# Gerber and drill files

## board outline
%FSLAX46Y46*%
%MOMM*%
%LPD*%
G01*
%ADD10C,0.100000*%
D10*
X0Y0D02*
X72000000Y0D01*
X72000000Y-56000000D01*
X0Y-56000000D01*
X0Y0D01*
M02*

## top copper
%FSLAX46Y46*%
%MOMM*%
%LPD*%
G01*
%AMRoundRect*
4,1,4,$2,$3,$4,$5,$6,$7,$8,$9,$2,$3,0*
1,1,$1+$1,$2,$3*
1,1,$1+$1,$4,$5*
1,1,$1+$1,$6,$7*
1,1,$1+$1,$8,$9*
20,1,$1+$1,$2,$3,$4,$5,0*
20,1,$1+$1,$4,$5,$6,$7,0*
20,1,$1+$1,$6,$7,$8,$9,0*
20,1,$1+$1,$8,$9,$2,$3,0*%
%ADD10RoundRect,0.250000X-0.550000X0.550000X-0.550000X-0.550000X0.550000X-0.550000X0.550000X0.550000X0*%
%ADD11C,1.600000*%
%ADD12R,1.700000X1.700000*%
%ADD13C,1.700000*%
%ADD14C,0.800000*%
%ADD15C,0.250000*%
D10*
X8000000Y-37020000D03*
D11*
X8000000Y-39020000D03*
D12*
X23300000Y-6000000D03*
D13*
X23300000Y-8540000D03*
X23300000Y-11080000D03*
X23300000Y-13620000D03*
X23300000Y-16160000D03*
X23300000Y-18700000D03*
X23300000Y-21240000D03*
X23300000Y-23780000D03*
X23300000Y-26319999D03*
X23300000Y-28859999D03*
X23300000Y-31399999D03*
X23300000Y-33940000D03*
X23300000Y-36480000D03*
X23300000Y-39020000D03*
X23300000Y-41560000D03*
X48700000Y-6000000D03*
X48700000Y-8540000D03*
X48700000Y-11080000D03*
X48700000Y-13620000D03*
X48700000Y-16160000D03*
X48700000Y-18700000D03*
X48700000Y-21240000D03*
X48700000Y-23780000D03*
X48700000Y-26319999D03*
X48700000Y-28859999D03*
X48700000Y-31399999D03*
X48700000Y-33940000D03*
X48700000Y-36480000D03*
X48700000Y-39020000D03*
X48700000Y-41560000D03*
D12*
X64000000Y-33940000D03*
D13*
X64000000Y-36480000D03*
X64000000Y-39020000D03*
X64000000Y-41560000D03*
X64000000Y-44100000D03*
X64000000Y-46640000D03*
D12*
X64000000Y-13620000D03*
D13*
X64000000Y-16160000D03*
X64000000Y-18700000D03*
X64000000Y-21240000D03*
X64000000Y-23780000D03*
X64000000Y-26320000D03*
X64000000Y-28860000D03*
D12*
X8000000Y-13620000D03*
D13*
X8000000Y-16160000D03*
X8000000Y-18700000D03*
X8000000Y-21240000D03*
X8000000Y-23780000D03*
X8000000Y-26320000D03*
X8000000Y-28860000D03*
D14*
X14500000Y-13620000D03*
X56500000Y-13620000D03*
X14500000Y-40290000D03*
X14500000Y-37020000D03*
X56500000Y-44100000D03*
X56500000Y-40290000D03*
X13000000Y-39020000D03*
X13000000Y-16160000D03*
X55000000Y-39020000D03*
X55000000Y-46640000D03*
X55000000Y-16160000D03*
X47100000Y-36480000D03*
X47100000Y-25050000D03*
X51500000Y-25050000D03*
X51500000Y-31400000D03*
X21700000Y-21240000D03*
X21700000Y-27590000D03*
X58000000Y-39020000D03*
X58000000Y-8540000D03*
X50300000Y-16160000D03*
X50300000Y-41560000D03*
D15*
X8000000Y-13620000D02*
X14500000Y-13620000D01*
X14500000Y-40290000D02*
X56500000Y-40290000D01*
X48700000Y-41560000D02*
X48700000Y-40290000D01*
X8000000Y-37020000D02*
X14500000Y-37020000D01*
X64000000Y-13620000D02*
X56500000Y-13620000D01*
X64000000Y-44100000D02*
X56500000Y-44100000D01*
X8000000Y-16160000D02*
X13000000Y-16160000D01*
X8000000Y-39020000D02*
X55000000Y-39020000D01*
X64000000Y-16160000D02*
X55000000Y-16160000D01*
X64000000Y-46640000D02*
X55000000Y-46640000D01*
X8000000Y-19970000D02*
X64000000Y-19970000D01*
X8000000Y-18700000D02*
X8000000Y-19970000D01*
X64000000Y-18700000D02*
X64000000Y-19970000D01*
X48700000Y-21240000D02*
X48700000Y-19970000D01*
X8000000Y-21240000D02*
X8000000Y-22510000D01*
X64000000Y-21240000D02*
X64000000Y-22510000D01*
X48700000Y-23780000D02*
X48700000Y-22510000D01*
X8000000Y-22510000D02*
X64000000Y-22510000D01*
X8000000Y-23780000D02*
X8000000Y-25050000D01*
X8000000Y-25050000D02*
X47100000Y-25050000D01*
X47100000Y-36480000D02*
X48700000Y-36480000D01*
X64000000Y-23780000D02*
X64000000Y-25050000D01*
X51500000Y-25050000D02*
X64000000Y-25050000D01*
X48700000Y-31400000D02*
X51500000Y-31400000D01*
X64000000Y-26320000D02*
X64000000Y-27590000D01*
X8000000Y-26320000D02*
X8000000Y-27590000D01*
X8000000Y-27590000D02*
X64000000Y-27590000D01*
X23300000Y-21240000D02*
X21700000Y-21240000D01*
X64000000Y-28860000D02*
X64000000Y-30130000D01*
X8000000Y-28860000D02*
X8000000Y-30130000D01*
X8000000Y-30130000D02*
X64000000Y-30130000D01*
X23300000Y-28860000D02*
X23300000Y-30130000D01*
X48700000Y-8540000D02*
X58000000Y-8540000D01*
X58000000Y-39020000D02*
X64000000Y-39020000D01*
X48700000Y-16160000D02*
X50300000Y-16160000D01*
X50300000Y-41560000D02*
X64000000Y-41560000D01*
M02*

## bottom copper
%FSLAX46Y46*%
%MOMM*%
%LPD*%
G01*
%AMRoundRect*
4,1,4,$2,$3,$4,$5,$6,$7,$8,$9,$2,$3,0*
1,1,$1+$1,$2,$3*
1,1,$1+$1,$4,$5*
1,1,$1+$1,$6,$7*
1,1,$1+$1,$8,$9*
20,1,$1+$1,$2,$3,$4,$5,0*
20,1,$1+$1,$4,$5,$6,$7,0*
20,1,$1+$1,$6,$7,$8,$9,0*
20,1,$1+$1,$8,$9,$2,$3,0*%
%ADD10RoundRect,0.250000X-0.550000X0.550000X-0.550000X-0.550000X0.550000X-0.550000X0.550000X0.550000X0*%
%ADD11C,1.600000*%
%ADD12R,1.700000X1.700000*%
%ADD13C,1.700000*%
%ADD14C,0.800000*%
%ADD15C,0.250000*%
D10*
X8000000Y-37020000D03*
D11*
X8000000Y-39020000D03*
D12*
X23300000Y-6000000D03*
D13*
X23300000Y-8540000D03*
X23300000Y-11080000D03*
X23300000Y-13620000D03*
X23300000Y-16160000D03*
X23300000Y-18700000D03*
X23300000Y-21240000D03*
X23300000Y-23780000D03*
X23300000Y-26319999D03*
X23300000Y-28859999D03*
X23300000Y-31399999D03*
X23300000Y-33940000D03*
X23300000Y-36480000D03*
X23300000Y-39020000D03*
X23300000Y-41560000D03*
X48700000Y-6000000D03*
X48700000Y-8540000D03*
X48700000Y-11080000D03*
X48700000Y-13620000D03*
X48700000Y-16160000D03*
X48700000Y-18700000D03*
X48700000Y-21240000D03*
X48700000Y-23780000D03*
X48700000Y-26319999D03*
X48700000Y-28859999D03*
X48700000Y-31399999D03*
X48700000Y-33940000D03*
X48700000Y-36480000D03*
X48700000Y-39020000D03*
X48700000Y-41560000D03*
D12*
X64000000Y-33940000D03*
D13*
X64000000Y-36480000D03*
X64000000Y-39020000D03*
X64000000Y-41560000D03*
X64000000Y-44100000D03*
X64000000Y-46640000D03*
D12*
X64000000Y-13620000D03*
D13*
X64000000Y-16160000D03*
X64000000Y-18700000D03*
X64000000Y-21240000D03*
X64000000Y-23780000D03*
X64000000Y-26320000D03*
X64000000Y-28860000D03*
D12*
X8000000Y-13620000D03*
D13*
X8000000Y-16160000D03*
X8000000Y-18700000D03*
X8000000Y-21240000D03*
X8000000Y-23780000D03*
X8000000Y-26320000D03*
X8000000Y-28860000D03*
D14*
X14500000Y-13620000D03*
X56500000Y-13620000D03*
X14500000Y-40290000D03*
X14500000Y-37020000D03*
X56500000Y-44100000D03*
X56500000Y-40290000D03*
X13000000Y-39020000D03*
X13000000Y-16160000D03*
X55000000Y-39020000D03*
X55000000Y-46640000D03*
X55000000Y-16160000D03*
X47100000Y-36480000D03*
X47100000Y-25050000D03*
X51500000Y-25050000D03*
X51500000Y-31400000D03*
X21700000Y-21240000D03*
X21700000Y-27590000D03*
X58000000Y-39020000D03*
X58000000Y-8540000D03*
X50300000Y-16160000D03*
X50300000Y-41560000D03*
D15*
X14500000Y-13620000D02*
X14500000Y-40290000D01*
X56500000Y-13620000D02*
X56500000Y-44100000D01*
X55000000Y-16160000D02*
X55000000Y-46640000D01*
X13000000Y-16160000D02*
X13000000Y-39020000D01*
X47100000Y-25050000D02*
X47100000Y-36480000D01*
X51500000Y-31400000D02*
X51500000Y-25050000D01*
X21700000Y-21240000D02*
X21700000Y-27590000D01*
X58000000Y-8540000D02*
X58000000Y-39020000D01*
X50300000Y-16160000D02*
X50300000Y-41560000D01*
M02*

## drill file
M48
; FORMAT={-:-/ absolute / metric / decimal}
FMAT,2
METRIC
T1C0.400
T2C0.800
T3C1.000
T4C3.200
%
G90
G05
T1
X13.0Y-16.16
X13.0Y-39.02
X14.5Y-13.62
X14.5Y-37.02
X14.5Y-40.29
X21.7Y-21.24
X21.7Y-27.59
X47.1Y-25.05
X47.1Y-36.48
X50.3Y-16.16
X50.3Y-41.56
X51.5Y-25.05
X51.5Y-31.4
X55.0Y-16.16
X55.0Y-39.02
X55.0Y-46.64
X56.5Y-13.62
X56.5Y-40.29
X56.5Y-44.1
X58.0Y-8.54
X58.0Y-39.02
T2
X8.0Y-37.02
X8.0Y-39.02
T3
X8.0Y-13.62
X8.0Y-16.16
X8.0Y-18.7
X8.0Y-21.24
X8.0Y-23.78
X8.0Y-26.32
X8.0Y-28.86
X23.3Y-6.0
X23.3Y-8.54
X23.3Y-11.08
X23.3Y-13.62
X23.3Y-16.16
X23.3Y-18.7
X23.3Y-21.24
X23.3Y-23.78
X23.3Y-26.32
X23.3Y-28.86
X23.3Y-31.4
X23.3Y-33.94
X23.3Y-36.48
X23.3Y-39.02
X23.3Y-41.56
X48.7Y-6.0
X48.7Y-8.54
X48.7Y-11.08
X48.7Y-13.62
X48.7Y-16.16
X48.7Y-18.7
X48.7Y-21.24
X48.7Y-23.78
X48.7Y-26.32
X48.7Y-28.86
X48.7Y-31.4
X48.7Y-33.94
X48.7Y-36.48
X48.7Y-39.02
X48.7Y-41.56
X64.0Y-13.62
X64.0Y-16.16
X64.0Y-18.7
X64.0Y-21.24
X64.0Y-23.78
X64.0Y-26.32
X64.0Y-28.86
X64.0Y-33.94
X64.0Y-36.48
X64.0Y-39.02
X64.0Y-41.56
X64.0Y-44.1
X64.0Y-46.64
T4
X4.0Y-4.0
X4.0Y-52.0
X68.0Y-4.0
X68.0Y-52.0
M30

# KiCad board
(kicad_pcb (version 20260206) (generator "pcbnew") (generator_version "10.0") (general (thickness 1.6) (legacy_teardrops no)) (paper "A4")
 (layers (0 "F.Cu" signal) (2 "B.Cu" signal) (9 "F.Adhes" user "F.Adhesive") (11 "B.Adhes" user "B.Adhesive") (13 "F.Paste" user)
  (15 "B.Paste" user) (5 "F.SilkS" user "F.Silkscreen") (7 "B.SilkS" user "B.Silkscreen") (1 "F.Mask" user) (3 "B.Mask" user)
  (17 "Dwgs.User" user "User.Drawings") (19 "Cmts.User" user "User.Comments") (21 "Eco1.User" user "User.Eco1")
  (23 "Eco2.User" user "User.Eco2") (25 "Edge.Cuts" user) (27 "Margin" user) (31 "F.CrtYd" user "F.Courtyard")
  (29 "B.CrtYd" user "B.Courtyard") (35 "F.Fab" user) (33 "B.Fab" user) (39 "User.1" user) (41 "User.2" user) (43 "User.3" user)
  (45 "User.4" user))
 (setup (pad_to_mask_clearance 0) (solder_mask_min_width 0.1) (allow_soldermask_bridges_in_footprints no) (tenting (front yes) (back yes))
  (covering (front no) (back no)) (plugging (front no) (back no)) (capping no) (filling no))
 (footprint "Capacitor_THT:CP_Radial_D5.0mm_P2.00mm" (layer "F.Cu") (at 8 37.02 -90)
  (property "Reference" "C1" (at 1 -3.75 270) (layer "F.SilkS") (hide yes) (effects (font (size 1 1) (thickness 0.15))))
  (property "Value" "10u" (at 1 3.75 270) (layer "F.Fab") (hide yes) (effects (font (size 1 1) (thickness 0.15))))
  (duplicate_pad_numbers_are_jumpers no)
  (pad "1" thru_hole roundrect (at 0 0 270) (size 1.6 1.6) (drill 0.8) (layers "*.Cu" "*.Mask") (remove_unused_layers no)
   (roundrect_rratio 0.15625) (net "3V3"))
  (pad "2" thru_hole circle (at 2 0 270) (size 1.6 1.6) (drill 0.8) (layers "*.Cu" "*.Mask") (remove_unused_layers no) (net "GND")))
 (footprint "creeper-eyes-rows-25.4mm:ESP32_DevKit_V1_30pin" (layer "F.Cu") (at 36 23.78)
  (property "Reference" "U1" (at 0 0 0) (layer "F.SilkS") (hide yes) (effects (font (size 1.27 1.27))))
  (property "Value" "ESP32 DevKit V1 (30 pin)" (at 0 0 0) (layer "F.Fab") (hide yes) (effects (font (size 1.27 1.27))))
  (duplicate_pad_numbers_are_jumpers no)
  (pad "1" thru_hole rect (at -12.7 -17.78) (size 1.7 1.7) (drill 1) (layers "*.Cu" "*.Mask") (remove_unused_layers no)
   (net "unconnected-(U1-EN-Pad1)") (thermal_bridge_angle 45))
  (pad "2" thru_hole circle (at -12.7 -15.24) (size 1.7 1.7) (drill 1) (layers "*.Cu" "*.Mask") (remove_unused_layers no)
   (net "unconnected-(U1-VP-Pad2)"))
  (pad "3" thru_hole circle (at -12.7 -12.7) (size 1.7 1.7) (drill 1) (layers "*.Cu" "*.Mask") (remove_unused_layers no)
   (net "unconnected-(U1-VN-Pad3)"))
  (pad "4" thru_hole circle (at -12.7 -10.16) (size 1.7 1.7) (drill 1) (layers "*.Cu" "*.Mask") (remove_unused_layers no)
   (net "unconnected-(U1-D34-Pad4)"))
  (pad "5" thru_hole circle (at -12.7 -7.62) (size 1.7 1.7) (drill 1) (layers "*.Cu" "*.Mask") (remove_unused_layers no)
   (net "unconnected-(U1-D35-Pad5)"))
  (pad "6" thru_hole circle (at -12.7 -5.08) (size 1.7 1.7) (drill 1) (layers "*.Cu" "*.Mask") (remove_unused_layers no)
   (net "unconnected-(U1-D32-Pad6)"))
  (pad "7" thru_hole circle (at -12.7 -2.54) (size 1.7 1.7) (drill 1) (layers "*.Cu" "*.Mask") (remove_unused_layers no) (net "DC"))
  (pad "8" thru_hole circle (at -12.7 0) (size 1.7 1.7) (drill 1) (layers "*.Cu" "*.Mask") (remove_unused_layers no)
   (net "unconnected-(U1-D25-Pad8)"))
  (pad "9" thru_hole circle (at -12.7 2.539999) (size 1.7 1.7) (drill 1) (layers "*.Cu" "*.Mask") (remove_unused_layers no)
   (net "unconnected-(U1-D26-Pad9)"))
  (pad "10" thru_hole circle (at -12.7 5.079999) (size 1.7 1.7) (drill 1) (layers "*.Cu" "*.Mask") (remove_unused_layers no) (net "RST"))
  (pad "11" thru_hole circle (at -12.7 7.619999) (size 1.7 1.7) (drill 1) (layers "*.Cu" "*.Mask") (remove_unused_layers no)
   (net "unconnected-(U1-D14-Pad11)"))
  (pad "12" thru_hole circle (at -12.7 10.16) (size 1.7 1.7) (drill 1) (layers "*.Cu" "*.Mask") (remove_unused_layers no)
   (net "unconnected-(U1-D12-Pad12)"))
  (pad "13" thru_hole circle (at -12.7 12.7) (size 1.7 1.7) (drill 1) (layers "*.Cu" "*.Mask") (remove_unused_layers no)
   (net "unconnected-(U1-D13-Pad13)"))
  (pad "14" thru_hole circle (at -12.7 15.24) (size 1.7 1.7) (drill 1) (layers "*.Cu" "*.Mask") (remove_unused_layers no) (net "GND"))
  (pad "15" thru_hole circle (at -12.7 17.78) (size 1.7 1.7) (drill 1) (layers "*.Cu" "*.Mask") (remove_unused_layers no)
   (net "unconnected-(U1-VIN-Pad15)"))
  (pad "16" thru_hole circle (at 12.7 -17.78) (size 1.7 1.7) (drill 1) (layers "*.Cu" "*.Mask") (remove_unused_layers no)
   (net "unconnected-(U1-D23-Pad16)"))
  (pad "17" thru_hole circle (at 12.7 -15.24) (size 1.7 1.7) (drill 1) (layers "*.Cu" "*.Mask") (remove_unused_layers no) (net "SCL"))
  (pad "18" thru_hole circle (at 12.7 -12.7) (size 1.7 1.7) (drill 1) (layers "*.Cu" "*.Mask") (remove_unused_layers no)
   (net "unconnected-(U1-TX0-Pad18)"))
  (pad "19" thru_hole circle (at 12.7 -10.16) (size 1.7 1.7) (drill 1) (layers "*.Cu" "*.Mask") (remove_unused_layers no)
   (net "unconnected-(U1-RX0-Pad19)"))
  (pad "20" thru_hole circle (at 12.7 -7.62) (size 1.7 1.7) (drill 1) (layers "*.Cu" "*.Mask") (remove_unused_layers no) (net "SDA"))
  (pad "21" thru_hole circle (at 12.7 -5.08) (size 1.7 1.7) (drill 1) (layers "*.Cu" "*.Mask") (remove_unused_layers no)
   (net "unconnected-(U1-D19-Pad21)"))
  (pad "22" thru_hole circle (at 12.7 -2.54) (size 1.7 1.7) (drill 1) (layers "*.Cu" "*.Mask") (remove_unused_layers no) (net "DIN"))
  (pad "23" thru_hole circle (at 12.7 0) (size 1.7 1.7) (drill 1) (layers "*.Cu" "*.Mask") (remove_unused_layers no) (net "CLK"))
  (pad "24" thru_hole circle (at 12.7 2.539999) (size 1.7 1.7) (drill 1) (layers "*.Cu" "*.Mask") (remove_unused_layers no)
   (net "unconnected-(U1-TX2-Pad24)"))
  (pad "25" thru_hole circle (at 12.7 5.079999) (size 1.7 1.7) (drill 1) (layers "*.Cu" "*.Mask") (remove_unused_layers no)
   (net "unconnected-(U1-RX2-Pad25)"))
  (pad "26" thru_hole circle (at 12.7 7.619999) (size 1.7 1.7) (drill 1) (layers "*.Cu" "*.Mask") (remove_unused_layers no) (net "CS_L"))
  (pad "27" thru_hole circle (at 12.7 10.16) (size 1.7 1.7) (drill 1) (layers "*.Cu" "*.Mask") (remove_unused_layers no)
   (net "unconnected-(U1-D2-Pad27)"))
  (pad "28" thru_hole circle (at 12.7 12.7) (size 1.7 1.7) (drill 1) (layers "*.Cu" "*.Mask") (remove_unused_layers no) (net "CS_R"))
  (pad "29" thru_hole circle (at 12.7 15.24) (size 1.7 1.7) (drill 1) (layers "*.Cu" "*.Mask") (remove_unused_layers no) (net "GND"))
  (pad "30" thru_hole circle (at 12.7 17.78) (size 1.7 1.7) (drill 1) (layers "*.Cu" "*.Mask") (remove_unused_layers no) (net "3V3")))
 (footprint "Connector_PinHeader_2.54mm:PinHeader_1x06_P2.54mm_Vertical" (layer "F.Cu") (at 64 33.94)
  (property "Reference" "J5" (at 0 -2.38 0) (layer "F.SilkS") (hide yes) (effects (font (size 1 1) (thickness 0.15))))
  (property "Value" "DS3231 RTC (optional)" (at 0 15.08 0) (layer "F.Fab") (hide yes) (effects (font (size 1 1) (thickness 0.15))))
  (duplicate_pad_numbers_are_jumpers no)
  (pad "1" thru_hole rect (at 0 0) (size 1.7 1.7) (drill 1) (layers "*.Cu" "*.Mask") (remove_unused_layers no)
   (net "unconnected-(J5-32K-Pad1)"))
  (pad "2" thru_hole circle (at 0 2.54) (size 1.7 1.7) (drill 1) (layers "*.Cu" "*.Mask") (remove_unused_layers no)
   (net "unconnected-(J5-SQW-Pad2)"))
  (pad "3" thru_hole circle (at 0 5.08) (size 1.7 1.7) (drill 1) (layers "*.Cu" "*.Mask") (remove_unused_layers no) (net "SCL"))
  (pad "4" thru_hole circle (at 0 7.62) (size 1.7 1.7) (drill 1) (layers "*.Cu" "*.Mask") (remove_unused_layers no) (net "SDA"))
  (pad "5" thru_hole circle (at 0 10.16) (size 1.7 1.7) (drill 1) (layers "*.Cu" "*.Mask") (remove_unused_layers no) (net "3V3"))
  (pad "6" thru_hole circle (at 0 12.7) (size 1.7 1.7) (drill 1) (layers "*.Cu" "*.Mask") (remove_unused_layers no) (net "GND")))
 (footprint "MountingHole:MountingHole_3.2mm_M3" (layer "F.Cu") (at 4 4)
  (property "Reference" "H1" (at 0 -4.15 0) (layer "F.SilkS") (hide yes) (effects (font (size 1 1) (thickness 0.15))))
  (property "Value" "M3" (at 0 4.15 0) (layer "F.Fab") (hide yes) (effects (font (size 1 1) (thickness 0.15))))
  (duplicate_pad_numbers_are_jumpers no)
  (pad "" np_thru_hole circle (at 0 0) (size 3.2 3.2) (drill 3.2) (layers "*.Cu" "*.Mask")))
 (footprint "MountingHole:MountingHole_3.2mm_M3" (layer "F.Cu") (at 68 52)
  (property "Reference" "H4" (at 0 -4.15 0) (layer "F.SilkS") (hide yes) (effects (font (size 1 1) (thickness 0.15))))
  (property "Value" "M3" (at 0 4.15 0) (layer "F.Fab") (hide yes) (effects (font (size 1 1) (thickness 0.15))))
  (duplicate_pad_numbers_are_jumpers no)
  (pad "" np_thru_hole circle (at 0 0) (size 3.2 3.2) (drill 3.2) (layers "*.Cu" "*.Mask")))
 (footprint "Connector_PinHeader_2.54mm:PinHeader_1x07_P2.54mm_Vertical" (layer "F.Cu") (at 64 13.62)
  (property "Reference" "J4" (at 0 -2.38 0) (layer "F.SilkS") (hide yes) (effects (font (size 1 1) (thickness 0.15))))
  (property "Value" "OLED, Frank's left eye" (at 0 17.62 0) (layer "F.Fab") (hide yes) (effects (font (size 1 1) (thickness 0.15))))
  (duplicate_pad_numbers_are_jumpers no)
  (pad "1" thru_hole rect (at 0 0) (size 1.7 1.7) (drill 1) (layers "*.Cu" "*.Mask") (remove_unused_layers no) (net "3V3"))
  (pad "2" thru_hole circle (at 0 2.54) (size 1.7 1.7) (drill 1) (layers "*.Cu" "*.Mask") (remove_unused_layers no) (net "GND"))
  (pad "3" thru_hole circle (at 0 5.08) (size 1.7 1.7) (drill 1) (layers "*.Cu" "*.Mask") (remove_unused_layers no) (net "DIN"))
  (pad "4" thru_hole circle (at 0 7.62) (size 1.7 1.7) (drill 1) (layers "*.Cu" "*.Mask") (remove_unused_layers no) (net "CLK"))
  (pad "5" thru_hole circle (at 0 10.16) (size 1.7 1.7) (drill 1) (layers "*.Cu" "*.Mask") (remove_unused_layers no) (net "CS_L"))
  (pad "6" thru_hole circle (at 0 12.7) (size 1.7 1.7) (drill 1) (layers "*.Cu" "*.Mask") (remove_unused_layers no) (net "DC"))
  (pad "7" thru_hole circle (at 0 15.24) (size 1.7 1.7) (drill 1) (layers "*.Cu" "*.Mask") (remove_unused_layers no) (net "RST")))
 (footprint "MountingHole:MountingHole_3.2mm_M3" (layer "F.Cu") (at 68 4)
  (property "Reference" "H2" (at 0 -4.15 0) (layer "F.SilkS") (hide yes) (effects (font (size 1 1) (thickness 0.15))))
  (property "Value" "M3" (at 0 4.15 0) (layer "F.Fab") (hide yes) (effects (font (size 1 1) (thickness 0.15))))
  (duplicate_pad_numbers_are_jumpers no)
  (pad "" np_thru_hole circle (at 0 0) (size 3.2 3.2) (drill 3.2) (layers "*.Cu" "*.Mask")))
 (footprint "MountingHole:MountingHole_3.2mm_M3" (layer "F.Cu") (at 4 52)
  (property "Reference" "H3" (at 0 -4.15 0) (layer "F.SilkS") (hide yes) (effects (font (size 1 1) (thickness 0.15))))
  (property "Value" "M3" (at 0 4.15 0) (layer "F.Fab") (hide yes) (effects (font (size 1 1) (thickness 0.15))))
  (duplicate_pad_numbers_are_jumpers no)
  (pad "" np_thru_hole circle (at 0 0) (size 3.2 3.2) (drill 3.2) (layers "*.Cu" "*.Mask")))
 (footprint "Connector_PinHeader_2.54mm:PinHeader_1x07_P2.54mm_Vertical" (layer "F.Cu") (at 8 13.62)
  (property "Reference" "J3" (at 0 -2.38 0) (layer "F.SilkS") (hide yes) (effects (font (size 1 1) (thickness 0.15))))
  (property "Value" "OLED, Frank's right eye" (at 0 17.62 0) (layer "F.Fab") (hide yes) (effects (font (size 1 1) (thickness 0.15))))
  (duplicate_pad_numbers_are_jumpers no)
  (pad "1" thru_hole rect (at 0 0) (size 1.7 1.7) (drill 1) (layers "*.Cu" "*.Mask") (remove_unused_layers no) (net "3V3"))
  (pad "2" thru_hole circle (at 0 2.54) (size 1.7 1.7) (drill 1) (layers "*.Cu" "*.Mask") (remove_unused_layers no) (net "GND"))
  (pad "3" thru_hole circle (at 0 5.08) (size 1.7 1.7) (drill 1) (layers "*.Cu" "*.Mask") (remove_unused_layers no) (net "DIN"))
  (pad "4" thru_hole circle (at 0 7.62) (size 1.7 1.7) (drill 1) (layers "*.Cu" "*.Mask") (remove_unused_layers no) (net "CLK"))
  (pad "5" thru_hole circle (at 0 10.16) (size 1.7 1.7) (drill 1) (layers "*.Cu" "*.Mask") (remove_unused_layers no) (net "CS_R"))
  (pad "6" thru_hole circle (at 0 12.7) (size 1.7 1.7) (drill 1) (layers "*.Cu" "*.Mask") (remove_unused_layers no) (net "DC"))
  (pad "7" thru_hole circle (at 0 15.24) (size 1.7 1.7) (drill 1) (layers "*.Cu" "*.Mask") (remove_unused_layers no) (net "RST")))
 (gr_rect (start 0 0) (end 72 56) (stroke (width 0.1) (type default)) (fill no) (layer "Edge.Cuts"))
 (segment (start 8 13.62) (end 14.5 13.62) (width 0.25) (layer "F.Cu") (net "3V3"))
 (segment (start 14.5 40.29) (end 56.5 40.29) (width 0.25) (layer "F.Cu") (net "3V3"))
 (segment (start 48.7 41.56) (end 48.7 40.29) (width 0.25) (layer "F.Cu") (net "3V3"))
 (segment (start 8 37.02) (end 14.5 37.02) (width 0.25) (layer "F.Cu") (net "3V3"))
 (segment (start 64 13.62) (end 56.5 13.62) (width 0.25) (layer "F.Cu") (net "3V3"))
 (segment (start 64 44.1) (end 56.5 44.1) (width 0.25) (layer "F.Cu") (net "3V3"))
 (via (at 14.5 13.62) (size 0.8) (drill 0.4) (layers "F.Cu" "B.Cu") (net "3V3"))
 (via (at 56.5 13.62) (size 0.8) (drill 0.4) (layers "F.Cu" "B.Cu") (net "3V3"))
 (via (at 14.5 40.29) (size 0.8) (drill 0.4) (layers "F.Cu" "B.Cu") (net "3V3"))
 (via (at 14.5 37.02) (size 0.8) (drill 0.4) (layers "F.Cu" "B.Cu") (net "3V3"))
 (via (at 56.5 44.1) (size 0.8) (drill 0.4) (layers "F.Cu" "B.Cu") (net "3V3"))
 (via (at 56.5 40.29) (size 0.8) (drill 0.4) (layers "F.Cu" "B.Cu") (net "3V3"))
 (segment (start 14.5 13.62) (end 14.5 40.29) (width 0.25) (layer "B.Cu") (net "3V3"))
 (segment (start 56.5 13.62) (end 56.5 44.1) (width 0.25) (layer "B.Cu") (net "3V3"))
 (segment (start 8 16.16) (end 13 16.16) (width 0.25) (layer "F.Cu") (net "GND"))
 (segment (start 8 39.02) (end 55 39.02) (width 0.25) (layer "F.Cu") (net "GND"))
 (segment (start 64 16.16) (end 55 16.16) (width 0.25) (layer "F.Cu") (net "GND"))
 (segment (start 64 46.64) (end 55 46.64) (width 0.25) (layer "F.Cu") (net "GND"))
 (via (at 13 39.02) (size 0.8) (drill 0.4) (layers "F.Cu" "B.Cu") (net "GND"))
 (via (at 13 16.16) (size 0.8) (drill 0.4) (layers "F.Cu" "B.Cu") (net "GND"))
 (via (at 55 39.02) (size 0.8) (drill 0.4) (layers "F.Cu" "B.Cu") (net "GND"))
 (via (at 55 46.64) (size 0.8) (drill 0.4) (layers "F.Cu" "B.Cu") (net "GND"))
 (via (at 55 16.16) (size 0.8) (drill 0.4) (layers "F.Cu" "B.Cu") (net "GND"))
 (segment (start 55 16.16) (end 55 46.64) (width 0.25) (layer "B.Cu") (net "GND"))
 (segment (start 13 16.16) (end 13 39.02) (width 0.25) (layer "B.Cu") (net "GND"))
 (segment (start 8 19.97) (end 64 19.97) (width 0.25) (layer "F.Cu") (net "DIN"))
 (segment (start 8 18.7) (end 8 19.97) (width 0.25) (layer "F.Cu") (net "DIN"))
 (segment (start 64 18.7) (end 64 19.97) (width 0.25) (layer "F.Cu") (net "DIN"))
 (segment (start 48.7 21.24) (end 48.7 19.97) (width 0.25) (layer "F.Cu") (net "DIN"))
 (segment (start 8 21.24) (end 8 22.51) (width 0.25) (layer "F.Cu") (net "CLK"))
 (segment (start 64 21.24) (end 64 22.51) (width 0.25) (layer "F.Cu") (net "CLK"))
 (segment (start 48.7 23.78) (end 48.7 22.51) (width 0.25) (layer "F.Cu") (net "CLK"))
 (segment (start 8 22.51) (end 64 22.51) (width 0.25) (layer "F.Cu") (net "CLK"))
 (segment (start 8 23.78) (end 8 25.05) (width 0.25) (layer "F.Cu") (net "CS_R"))
 (segment (start 8 25.05) (end 47.1 25.05) (width 0.25) (layer "F.Cu") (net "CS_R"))
 (segment (start 47.1 36.48) (end 48.7 36.48) (width 0.25) (layer "F.Cu") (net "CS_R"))
 (via (at 47.1 36.48) (size 0.8) (drill 0.4) (layers "F.Cu" "B.Cu") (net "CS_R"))
 (via (at 47.1 25.05) (size 0.8) (drill 0.4) (layers "F.Cu" "B.Cu") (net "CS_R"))
 (segment (start 47.1 25.05) (end 47.1 36.48) (width 0.25) (layer "B.Cu") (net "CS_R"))
 (segment (start 64 23.78) (end 64 25.05) (width 0.25) (layer "F.Cu") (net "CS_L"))
 (segment (start 51.5 25.05) (end 64 25.05) (width 0.25) (layer "F.Cu") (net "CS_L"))
 (segment (start 48.7 31.4) (end 51.5 31.4) (width 0.25) (layer "F.Cu") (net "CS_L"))
 (via (at 51.5 25.05) (size 0.8) (drill 0.4) (layers "F.Cu" "B.Cu") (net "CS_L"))
 (via (at 51.5 31.4) (size 0.8) (drill 0.4) (layers "F.Cu" "B.Cu") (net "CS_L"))
 (segment (start 51.5 31.4) (end 51.5 25.05) (width 0.25) (layer "B.Cu") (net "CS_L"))
 (segment (start 64 26.32) (end 64 27.59) (width 0.25) (layer "F.Cu") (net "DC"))
 (segment (start 8 26.32) (end 8 27.59) (width 0.25) (layer "F.Cu") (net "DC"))
 (segment (start 8 27.59) (end 64 27.59) (width 0.25) (layer "F.Cu") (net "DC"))
 (segment (start 23.3 21.24) (end 21.7 21.24) (width 0.25) (layer "F.Cu") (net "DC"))
 (via (at 21.7 21.24) (size 0.8) (drill 0.4) (layers "F.Cu" "B.Cu") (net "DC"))
 (via (at 21.7 27.59) (size 0.8) (drill 0.4) (layers "F.Cu" "B.Cu") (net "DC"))
 (segment (start 21.7 21.24) (end 21.7 27.59) (width 0.25) (layer "B.Cu") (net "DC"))
 (segment (start 64 28.86) (end 64 30.13) (width 0.25) (layer "F.Cu") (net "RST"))
 (segment (start 8 28.86) (end 8 30.13) (width 0.25) (layer "F.Cu") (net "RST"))
 (segment (start 8 30.13) (end 64 30.13) (width 0.25) (layer "F.Cu") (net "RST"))
 (segment (start 23.3 28.86) (end 23.3 30.13) (width 0.25) (layer "F.Cu") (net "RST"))
 (segment (start 48.7 8.54) (end 58 8.54) (width 0.25) (layer "F.Cu") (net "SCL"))
 (segment (start 58 39.02) (end 64 39.02) (width 0.25) (layer "F.Cu") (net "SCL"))
 (via (at 58 39.02) (size 0.8) (drill 0.4) (layers "F.Cu" "B.Cu") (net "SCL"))
 (via (at 58 8.54) (size 0.8) (drill 0.4) (layers "F.Cu" "B.Cu") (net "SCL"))
 (segment (start 58 8.54) (end 58 39.02) (width 0.25) (layer "B.Cu") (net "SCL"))
 (segment (start 48.7 16.16) (end 50.3 16.16) (width 0.25) (layer "F.Cu") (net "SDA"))
 (segment (start 50.3 41.56) (end 64 41.56) (width 0.25) (layer "F.Cu") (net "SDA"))
 (via (at 50.3 16.16) (size 0.8) (drill 0.4) (layers "F.Cu" "B.Cu") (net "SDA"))
 (via (at 50.3 41.56) (size 0.8) (drill 0.4) (layers "F.Cu" "B.Cu") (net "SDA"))
 (segment (start 50.3 16.16) (end 50.3 41.56) (width 0.25) (layer "B.Cu") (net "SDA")))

